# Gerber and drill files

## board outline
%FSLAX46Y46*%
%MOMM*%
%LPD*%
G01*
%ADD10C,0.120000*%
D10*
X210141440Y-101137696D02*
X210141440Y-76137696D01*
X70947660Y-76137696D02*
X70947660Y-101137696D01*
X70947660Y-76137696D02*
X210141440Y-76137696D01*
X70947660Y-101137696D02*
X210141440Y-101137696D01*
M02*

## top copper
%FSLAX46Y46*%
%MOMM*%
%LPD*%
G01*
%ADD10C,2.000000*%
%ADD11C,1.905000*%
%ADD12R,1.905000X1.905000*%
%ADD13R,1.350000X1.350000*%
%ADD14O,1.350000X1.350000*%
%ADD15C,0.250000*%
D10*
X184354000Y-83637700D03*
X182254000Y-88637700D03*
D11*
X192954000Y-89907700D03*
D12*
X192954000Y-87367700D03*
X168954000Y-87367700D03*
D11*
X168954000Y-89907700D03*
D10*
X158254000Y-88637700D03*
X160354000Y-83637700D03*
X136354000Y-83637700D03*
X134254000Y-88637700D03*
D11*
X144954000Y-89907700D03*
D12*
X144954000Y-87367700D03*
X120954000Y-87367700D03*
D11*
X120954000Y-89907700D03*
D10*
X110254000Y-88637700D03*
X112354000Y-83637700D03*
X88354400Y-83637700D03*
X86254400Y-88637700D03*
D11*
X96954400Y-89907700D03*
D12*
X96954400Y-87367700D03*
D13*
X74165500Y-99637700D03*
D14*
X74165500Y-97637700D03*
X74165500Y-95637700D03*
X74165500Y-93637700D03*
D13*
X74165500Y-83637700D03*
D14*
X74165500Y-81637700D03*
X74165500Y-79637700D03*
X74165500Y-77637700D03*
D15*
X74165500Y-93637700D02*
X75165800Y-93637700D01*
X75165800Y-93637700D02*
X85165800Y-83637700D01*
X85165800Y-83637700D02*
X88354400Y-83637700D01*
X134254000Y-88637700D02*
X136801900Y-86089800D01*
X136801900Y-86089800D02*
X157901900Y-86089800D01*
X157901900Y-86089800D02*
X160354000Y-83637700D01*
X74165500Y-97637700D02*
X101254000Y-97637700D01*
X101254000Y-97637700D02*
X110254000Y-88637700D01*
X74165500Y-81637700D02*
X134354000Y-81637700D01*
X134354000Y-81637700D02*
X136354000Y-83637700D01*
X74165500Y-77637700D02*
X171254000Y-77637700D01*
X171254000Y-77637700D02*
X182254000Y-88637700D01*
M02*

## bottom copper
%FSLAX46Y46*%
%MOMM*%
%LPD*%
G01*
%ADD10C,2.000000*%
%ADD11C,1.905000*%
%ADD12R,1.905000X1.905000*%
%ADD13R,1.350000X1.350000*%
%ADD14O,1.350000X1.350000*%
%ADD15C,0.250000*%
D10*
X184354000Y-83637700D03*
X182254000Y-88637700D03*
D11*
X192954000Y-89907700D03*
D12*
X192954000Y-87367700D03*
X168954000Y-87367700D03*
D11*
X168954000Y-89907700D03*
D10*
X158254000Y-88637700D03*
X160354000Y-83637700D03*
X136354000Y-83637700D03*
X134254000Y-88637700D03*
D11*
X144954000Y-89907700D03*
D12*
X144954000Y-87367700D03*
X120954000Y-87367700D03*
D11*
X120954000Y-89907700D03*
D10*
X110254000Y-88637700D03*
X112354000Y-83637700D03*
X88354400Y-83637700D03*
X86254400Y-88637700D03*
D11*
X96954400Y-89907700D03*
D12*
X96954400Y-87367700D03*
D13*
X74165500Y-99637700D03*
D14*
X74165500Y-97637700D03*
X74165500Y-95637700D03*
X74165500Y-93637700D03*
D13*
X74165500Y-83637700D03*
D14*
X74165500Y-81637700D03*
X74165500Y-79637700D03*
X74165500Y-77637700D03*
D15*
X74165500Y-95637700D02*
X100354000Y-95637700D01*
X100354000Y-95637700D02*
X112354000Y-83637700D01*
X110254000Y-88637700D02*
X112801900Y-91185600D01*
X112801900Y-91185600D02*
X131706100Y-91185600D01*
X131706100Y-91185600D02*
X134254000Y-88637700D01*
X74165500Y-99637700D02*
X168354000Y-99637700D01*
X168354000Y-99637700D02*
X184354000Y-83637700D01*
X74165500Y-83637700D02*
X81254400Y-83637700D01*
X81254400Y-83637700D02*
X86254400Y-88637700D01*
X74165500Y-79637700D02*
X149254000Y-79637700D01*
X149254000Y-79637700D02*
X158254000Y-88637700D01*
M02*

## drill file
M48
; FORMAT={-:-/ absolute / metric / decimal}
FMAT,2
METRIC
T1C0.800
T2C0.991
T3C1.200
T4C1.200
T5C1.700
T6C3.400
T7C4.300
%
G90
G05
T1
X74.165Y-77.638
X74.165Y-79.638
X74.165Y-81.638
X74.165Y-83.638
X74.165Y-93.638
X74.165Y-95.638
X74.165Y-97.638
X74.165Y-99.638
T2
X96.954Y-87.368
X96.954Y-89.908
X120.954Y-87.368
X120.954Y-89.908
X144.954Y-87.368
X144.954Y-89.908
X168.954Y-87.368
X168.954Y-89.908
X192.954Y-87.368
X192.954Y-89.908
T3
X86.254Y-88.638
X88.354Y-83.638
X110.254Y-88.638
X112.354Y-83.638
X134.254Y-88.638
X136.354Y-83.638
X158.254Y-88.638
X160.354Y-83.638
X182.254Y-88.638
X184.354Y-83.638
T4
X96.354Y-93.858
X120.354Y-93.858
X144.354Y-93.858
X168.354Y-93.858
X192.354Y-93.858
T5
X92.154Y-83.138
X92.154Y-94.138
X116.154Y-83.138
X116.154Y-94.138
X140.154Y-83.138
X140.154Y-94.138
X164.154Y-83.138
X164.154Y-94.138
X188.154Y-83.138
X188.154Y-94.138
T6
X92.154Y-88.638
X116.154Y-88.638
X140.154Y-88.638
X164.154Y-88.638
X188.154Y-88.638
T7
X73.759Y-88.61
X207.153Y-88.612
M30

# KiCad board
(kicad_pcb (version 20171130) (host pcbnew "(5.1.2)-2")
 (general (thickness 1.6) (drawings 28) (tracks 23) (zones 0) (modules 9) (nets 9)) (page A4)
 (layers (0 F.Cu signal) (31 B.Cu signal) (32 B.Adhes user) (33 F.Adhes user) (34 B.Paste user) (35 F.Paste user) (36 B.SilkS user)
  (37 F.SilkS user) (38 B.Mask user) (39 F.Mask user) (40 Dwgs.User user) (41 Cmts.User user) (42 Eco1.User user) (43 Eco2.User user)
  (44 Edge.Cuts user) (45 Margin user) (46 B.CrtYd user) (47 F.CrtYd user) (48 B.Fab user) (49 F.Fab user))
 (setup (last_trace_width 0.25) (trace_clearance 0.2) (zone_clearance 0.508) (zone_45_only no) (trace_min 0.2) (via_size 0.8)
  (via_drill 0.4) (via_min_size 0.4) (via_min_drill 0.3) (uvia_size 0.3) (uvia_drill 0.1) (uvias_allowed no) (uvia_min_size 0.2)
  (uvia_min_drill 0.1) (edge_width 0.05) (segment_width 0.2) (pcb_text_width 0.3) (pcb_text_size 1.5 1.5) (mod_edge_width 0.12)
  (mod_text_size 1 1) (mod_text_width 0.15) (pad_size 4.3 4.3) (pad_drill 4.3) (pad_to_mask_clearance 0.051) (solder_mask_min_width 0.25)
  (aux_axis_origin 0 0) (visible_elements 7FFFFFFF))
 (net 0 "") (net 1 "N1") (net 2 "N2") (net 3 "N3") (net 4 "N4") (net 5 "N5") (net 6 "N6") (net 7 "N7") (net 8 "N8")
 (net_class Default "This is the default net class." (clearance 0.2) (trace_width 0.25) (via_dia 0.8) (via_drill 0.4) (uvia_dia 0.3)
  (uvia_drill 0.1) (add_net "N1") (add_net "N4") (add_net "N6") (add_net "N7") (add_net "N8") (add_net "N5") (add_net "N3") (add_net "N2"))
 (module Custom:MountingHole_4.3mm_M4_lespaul (layer F.Cu) (at 205.812 88.6121)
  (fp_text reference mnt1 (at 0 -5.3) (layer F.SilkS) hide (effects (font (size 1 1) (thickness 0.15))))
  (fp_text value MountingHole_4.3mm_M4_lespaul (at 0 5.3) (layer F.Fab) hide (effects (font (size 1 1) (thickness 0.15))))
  (pad "" np_thru_hole circle (at 1.34138 0) (size 4.3 4.3) (drill 4.3) (layers *.Cu *.Mask)))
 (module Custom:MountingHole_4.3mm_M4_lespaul (layer F.Cu) (at 67.1085 86.4616)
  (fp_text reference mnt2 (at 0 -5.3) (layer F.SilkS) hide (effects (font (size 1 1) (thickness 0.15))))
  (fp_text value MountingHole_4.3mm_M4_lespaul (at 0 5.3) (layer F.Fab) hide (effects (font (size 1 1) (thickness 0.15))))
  (pad "" np_thru_hole circle (at 6.65026 2.14884) (size 4.3 4.3) (drill 4.3) (layers *.Cu *.Mask)))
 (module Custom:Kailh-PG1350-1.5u (layer F.Cu) (at 188.154 88.6377 270)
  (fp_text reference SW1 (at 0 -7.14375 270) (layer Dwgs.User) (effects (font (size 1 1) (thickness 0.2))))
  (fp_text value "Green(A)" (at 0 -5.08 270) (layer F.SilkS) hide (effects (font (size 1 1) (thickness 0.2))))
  (pad "" np_thru_hole circle (at 5.5 0 90) (size 1.7 1.7) (drill 1.7) (layers *.Cu *.Mask))
  (pad "" np_thru_hole circle (at -5.5 0 90) (size 1.7 1.7) (drill 1.7) (layers *.Cu *.Mask))
  (pad 2 thru_hole circle (at -5 3.8 311.9) (size 2 2) (drill 1.2) (layers *.Cu *.Mask) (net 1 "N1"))
  (pad 1 thru_hole circle (at 0 5.9 90) (size 2 2) (drill 1.2) (layers *.Cu *.Mask) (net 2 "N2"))
  (pad 3 thru_hole circle (at 1.27 -4.8 90) (size 1.905 1.905) (drill 0.9906) (layers *.Cu *.Mask))
  (pad 4 thru_hole rect (at -1.27 -4.8 90) (size 1.905 1.905) (drill 0.9906) (layers *.Cu *.Mask))
  (pad "" np_thru_hole circle (at 0 0 90) (size 3.4 3.4) (drill 3.4) (layers *.Cu *.Mask))
  (pad "" np_thru_hole circle (at 5.22 -4.2 90) (size 1.2 1.2) (drill 1.2) (layers *.Cu *.Mask)))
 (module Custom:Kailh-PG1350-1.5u (layer F.Cu) (at 164.154 88.6377 270)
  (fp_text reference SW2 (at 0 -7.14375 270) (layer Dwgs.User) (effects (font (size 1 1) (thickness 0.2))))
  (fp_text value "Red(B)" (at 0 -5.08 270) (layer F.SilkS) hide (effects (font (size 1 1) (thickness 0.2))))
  (pad "" np_thru_hole circle (at 5.22 -4.2 90) (size 1.2 1.2) (drill 1.2) (layers *.Cu *.Mask))
  (pad "" np_thru_hole circle (at 0 0 90) (size 3.4 3.4) (drill 3.4) (layers *.Cu *.Mask))
  (pad 4 thru_hole rect (at -1.27 -4.8 90) (size 1.905 1.905) (drill 0.9906) (layers *.Cu *.Mask))
  (pad 3 thru_hole circle (at 1.27 -4.8 90) (size 1.905 1.905) (drill 0.9906) (layers *.Cu *.Mask))
  (pad 1 thru_hole circle (at 0 5.9 90) (size 2 2) (drill 1.2) (layers *.Cu *.Mask) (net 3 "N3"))
  (pad 2 thru_hole circle (at -5 3.8 311.9) (size 2 2) (drill 1.2) (layers *.Cu *.Mask) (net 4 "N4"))
  (pad "" np_thru_hole circle (at -5.5 0 90) (size 1.7 1.7) (drill 1.7) (layers *.Cu *.Mask))
  (pad "" np_thru_hole circle (at 5.5 0 90) (size 1.7 1.7) (drill 1.7) (layers *.Cu *.Mask)))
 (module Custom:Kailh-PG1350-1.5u (layer F.Cu) (at 140.154 88.6377 270)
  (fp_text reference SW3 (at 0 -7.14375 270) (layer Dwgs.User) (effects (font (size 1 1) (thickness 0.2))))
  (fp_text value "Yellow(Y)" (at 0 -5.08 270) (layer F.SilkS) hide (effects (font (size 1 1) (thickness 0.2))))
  (pad "" np_thru_hole circle (at 5.5 0 90) (size 1.7 1.7) (drill 1.7) (layers *.Cu *.Mask))
  (pad "" np_thru_hole circle (at -5.5 0 90) (size 1.7 1.7) (drill 1.7) (layers *.Cu *.Mask))
  (pad 2 thru_hole circle (at -5 3.8 311.9) (size 2 2) (drill 1.2) (layers *.Cu *.Mask) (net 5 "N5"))
  (pad 1 thru_hole circle (at 0 5.9 90) (size 2 2) (drill 1.2) (layers *.Cu *.Mask) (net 4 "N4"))
  (pad 3 thru_hole circle (at 1.27 -4.8 90) (size 1.905 1.905) (drill 0.9906) (layers *.Cu *.Mask))
  (pad 4 thru_hole rect (at -1.27 -4.8 90) (size 1.905 1.905) (drill 0.9906) (layers *.Cu *.Mask))
  (pad "" np_thru_hole circle (at 0 0 90) (size 3.4 3.4) (drill 3.4) (layers *.Cu *.Mask))
  (pad "" np_thru_hole circle (at 5.22 -4.2 90) (size 1.2 1.2) (drill 1.2) (layers *.Cu *.Mask)))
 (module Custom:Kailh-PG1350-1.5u (layer F.Cu) (at 116.154 88.6377 270)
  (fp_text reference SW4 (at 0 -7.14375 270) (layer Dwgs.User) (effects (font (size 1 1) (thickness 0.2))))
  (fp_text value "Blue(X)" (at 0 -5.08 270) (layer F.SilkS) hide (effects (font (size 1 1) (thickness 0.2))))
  (pad "" np_thru_hole circle (at 5.22 -4.2 90) (size 1.2 1.2) (drill 1.2) (layers *.Cu *.Mask))
  (pad "" np_thru_hole circle (at 0 0 90) (size 3.4 3.4) (drill 3.4) (layers *.Cu *.Mask))
  (pad 4 thru_hole rect (at -1.27 -4.8 90) (size 1.905 1.905) (drill 0.9906) (layers *.Cu *.Mask))
  (pad 3 thru_hole circle (at 1.27 -4.8 90) (size 1.905 1.905) (drill 0.9906) (layers *.Cu *.Mask))
  (pad 1 thru_hole circle (at 0 5.9 90) (size 2 2) (drill 1.2) (layers *.Cu *.Mask) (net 4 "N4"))
  (pad 2 thru_hole circle (at -5 3.8 311.9) (size 2 2) (drill 1.2) (layers *.Cu *.Mask) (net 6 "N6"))
  (pad "" np_thru_hole circle (at -5.5 0 90) (size 1.7 1.7) (drill 1.7) (layers *.Cu *.Mask))
  (pad "" np_thru_hole circle (at 5.5 0 90) (size 1.7 1.7) (drill 1.7) (layers *.Cu *.Mask)))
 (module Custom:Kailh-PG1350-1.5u (layer F.Cu) (at 92.1544 88.6377 270)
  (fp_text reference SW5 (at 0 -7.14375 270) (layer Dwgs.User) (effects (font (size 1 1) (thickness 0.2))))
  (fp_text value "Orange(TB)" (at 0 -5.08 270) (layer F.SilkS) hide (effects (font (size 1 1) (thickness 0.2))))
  (pad "" np_thru_hole circle (at 5.5 0 90) (size 1.7 1.7) (drill 1.7) (layers *.Cu *.Mask))
  (pad "" np_thru_hole circle (at -5.5 0 90) (size 1.7 1.7) (drill 1.7) (layers *.Cu *.Mask))
  (pad 2 thru_hole circle (at -5 3.8 311.9) (size 2 2) (drill 1.2) (layers *.Cu *.Mask) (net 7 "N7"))
  (pad 1 thru_hole circle (at 0 5.9 90) (size 2 2) (drill 1.2) (layers *.Cu *.Mask) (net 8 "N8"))
  (pad 3 thru_hole circle (at 1.27 -4.8 90) (size 1.905 1.905) (drill 0.9906) (layers *.Cu *.Mask))
  (pad 4 thru_hole rect (at -1.27 -4.8 90) (size 1.905 1.905) (drill 0.9906) (layers *.Cu *.Mask))
  (pad "" np_thru_hole circle (at 0 0 90) (size 3.4 3.4) (drill 3.4) (layers *.Cu *.Mask))
  (pad "" np_thru_hole circle (at 5.22 -4.2 90) (size 1.2 1.2) (drill 1.2) (layers *.Cu *.Mask)))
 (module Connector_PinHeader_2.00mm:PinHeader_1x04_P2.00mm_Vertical (layer F.Cu) (at 74.1655 99.6377 180)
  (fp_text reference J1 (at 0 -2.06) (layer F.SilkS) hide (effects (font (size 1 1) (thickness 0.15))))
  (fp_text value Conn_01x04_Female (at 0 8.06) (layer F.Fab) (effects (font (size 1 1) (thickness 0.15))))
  (pad 1 thru_hole rect (at 0 0 180) (size 1.35 1.35) (drill 0.8) (layers *.Cu *.Mask) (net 1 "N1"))
  (pad 2 thru_hole oval (at 0 2 180) (size 1.35 1.35) (drill 0.8) (layers *.Cu *.Mask) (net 4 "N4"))
  (pad 3 thru_hole oval (at 0 4 180) (size 1.35 1.35) (drill 0.8) (layers *.Cu *.Mask) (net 6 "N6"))
  (pad 4 thru_hole oval (at 0 6 180) (size 1.35 1.35) (drill 0.8) (layers *.Cu *.Mask) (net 7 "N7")))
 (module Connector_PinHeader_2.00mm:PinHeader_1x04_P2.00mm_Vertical (layer F.Cu) (at 74.1655 83.6377 180)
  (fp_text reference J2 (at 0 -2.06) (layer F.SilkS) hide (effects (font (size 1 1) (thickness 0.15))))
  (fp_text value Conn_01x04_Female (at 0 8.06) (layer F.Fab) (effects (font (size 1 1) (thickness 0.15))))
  (pad 1 thru_hole rect (at 0 0 180) (size 1.35 1.35) (drill 0.8) (layers *.Cu *.Mask) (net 8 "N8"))
  (pad 2 thru_hole oval (at 0 2 180) (size 1.35 1.35) (drill 0.8) (layers *.Cu *.Mask) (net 5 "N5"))
  (pad 3 thru_hole oval (at 0 4 180) (size 1.35 1.35) (drill 0.8) (layers *.Cu *.Mask) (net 3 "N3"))
  (pad 4 thru_hole oval (at 0 6 180) (size 1.35 1.35) (drill 0.8) (layers *.Cu *.Mask) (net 2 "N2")))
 (gr_line (start 210.14144 101.137696) (end 210.14144 76.137696) (layer Edge.Cuts) (width 0.12))
 (gr_line (start 70.94766 76.137696) (end 70.94766 101.137696) (layer Edge.Cuts) (width 0.12))
 (gr_line (start 70.94766 76.137696) (end 210.14144 76.137696) (layer Edge.Cuts) (width 0.12))
 (gr_line (start 70.94766 101.137696) (end 210.14144 101.137696) (layer Edge.Cuts) (width 0.12))
 (segment (start 74.1655 93.6377) (end 75.1658 93.6377) (width 0.25) (layer F.Cu) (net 7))
 (segment (start 75.1658 93.6377) (end 85.1658 83.6377) (width 0.25) (layer F.Cu) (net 7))
 (segment (start 85.1658 83.6377) (end 88.3544 83.6377) (width 0.25) (layer F.Cu) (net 7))
 (segment (start 74.1655 95.6377) (end 100.354 95.6377) (width 0.25) (layer B.Cu) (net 6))
 (segment (start 100.354 95.6377) (end 112.354 83.6377) (width 0.25) (layer B.Cu) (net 6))
 (segment (start 134.254 88.6377) (end 136.8019 86.0898) (width 0.25) (layer F.Cu) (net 4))
 (segment (start 136.8019 86.0898) (end 157.9019 86.0898) (width 0.25) (layer F.Cu) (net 4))
 (segment (start 157.9019 86.0898) (end 160.354 83.6377) (width 0.25) (layer F.Cu) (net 4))
 (segment (start 110.254 88.6377) (end 112.8019 91.1856) (width 0.25) (layer B.Cu) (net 4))
 (segment (start 112.8019 91.1856) (end 131.7061 91.1856) (width 0.25) (layer B.Cu) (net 4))
 (segment (start 131.7061 91.1856) (end 134.254 88.6377) (width 0.25) (layer B.Cu) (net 4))
 (segment (start 74.1655 97.6377) (end 101.254 97.6377) (width 0.25) (layer F.Cu) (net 4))
 (segment (start 101.254 97.6377) (end 110.254 88.6377) (width 0.25) (layer F.Cu) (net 4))
 (segment (start 74.1655 99.6377) (end 168.354 99.6377) (width 0.25) (layer B.Cu) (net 1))
 (segment (start 168.354 99.6377) (end 184.354 83.6377) (width 0.25) (layer B.Cu) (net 1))
 (segment (start 74.1655 83.6377) (end 81.2544 83.6377) (width 0.25) (layer B.Cu) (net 8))
 (segment (start 81.2544 83.6377) (end 86.2544 88.6377) (width 0.25) (layer B.Cu) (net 8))
 (segment (start 74.1655 81.6377) (end 134.354 81.6377) (width 0.25) (layer F.Cu) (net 5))
 (segment (start 134.354 81.6377) (end 136.354 83.6377) (width 0.25) (layer F.Cu) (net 5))
 (segment (start 74.1655 79.6377) (end 149.254 79.6377) (width 0.25) (layer B.Cu) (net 3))
 (segment (start 149.254 79.6377) (end 158.254 88.6377) (width 0.25) (layer B.Cu) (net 3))
 (segment (start 74.1655 77.6377) (end 171.254 77.6377) (width 0.25) (layer F.Cu) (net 2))
 (segment (start 171.254 77.6377) (end 182.254 88.6377) (width 0.25) (layer F.Cu) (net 2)))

